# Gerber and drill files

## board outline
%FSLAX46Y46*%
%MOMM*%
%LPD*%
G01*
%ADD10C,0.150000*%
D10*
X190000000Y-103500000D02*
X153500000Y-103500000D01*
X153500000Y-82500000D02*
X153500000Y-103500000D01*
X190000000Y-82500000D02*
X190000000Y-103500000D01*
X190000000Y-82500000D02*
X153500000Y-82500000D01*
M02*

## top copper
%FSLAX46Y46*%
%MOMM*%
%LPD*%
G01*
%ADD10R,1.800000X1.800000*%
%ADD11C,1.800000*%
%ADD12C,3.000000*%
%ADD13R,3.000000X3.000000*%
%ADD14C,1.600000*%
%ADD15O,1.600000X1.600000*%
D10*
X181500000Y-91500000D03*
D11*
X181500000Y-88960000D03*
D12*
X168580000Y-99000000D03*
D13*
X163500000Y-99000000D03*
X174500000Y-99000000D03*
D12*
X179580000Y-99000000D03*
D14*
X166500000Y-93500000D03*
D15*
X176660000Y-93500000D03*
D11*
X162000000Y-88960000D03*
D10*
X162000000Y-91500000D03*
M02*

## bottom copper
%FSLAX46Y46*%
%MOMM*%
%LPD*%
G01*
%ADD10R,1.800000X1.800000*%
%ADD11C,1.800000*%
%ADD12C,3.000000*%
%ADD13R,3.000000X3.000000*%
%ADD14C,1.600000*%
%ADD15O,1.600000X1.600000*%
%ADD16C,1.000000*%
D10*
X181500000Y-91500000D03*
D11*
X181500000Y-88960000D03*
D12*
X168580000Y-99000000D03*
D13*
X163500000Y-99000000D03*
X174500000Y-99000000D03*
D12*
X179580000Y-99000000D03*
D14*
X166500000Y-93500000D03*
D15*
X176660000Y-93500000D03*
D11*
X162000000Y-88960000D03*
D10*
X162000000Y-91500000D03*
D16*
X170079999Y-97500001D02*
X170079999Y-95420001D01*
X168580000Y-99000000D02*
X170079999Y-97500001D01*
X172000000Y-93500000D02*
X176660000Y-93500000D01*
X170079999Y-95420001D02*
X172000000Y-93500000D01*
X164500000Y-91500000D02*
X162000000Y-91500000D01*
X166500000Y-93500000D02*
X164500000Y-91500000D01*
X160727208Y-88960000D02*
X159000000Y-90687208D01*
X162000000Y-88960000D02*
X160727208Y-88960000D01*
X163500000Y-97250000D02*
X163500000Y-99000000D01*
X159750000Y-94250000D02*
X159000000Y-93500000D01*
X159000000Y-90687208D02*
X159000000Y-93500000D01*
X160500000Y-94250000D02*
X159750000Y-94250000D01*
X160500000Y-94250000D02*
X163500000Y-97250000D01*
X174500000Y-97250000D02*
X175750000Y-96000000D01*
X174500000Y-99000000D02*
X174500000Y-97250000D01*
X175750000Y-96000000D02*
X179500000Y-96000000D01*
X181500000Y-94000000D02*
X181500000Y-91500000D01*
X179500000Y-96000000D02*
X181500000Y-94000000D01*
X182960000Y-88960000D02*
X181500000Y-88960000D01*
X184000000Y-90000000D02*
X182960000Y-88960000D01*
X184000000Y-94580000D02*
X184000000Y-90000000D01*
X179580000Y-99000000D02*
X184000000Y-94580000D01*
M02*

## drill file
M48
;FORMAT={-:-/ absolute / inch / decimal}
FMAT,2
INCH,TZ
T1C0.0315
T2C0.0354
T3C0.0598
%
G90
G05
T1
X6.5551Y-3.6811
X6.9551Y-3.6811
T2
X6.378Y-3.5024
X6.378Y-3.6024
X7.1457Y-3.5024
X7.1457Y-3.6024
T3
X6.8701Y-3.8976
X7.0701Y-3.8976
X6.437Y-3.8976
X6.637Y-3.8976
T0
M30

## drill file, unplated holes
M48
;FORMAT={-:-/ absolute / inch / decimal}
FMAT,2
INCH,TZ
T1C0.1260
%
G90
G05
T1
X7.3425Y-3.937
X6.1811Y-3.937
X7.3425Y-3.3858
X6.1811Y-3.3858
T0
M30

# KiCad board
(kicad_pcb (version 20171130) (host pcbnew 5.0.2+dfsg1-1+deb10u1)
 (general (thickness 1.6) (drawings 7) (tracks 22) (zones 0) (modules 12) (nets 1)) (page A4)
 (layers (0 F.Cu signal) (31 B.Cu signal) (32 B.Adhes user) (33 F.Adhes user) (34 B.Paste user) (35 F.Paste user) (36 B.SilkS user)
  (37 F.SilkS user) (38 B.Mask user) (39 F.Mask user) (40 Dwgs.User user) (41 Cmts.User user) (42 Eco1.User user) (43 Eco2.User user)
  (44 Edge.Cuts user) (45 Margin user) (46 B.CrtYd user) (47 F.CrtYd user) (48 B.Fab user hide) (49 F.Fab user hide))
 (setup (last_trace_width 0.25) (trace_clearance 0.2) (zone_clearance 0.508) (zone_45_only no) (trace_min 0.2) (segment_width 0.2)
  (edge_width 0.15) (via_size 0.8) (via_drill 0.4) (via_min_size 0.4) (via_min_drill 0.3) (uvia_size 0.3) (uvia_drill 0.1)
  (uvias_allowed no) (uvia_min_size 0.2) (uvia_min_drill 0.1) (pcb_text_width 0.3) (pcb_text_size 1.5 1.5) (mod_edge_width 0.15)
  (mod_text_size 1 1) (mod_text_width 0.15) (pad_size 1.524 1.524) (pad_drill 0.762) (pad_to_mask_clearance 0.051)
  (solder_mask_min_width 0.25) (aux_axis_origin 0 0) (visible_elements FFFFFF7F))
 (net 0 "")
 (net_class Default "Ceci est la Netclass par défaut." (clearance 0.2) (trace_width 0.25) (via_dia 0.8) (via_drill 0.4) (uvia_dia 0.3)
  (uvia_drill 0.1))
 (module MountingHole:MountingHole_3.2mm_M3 (layer F.Cu) (at 157 100)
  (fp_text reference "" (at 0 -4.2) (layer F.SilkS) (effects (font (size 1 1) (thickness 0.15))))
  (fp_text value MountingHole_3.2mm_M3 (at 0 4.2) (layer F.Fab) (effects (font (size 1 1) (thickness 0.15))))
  (pad 1 np_thru_hole circle (at 0 0) (size 3.2 3.2) (drill 3.2) (layers *.Cu *.Mask)))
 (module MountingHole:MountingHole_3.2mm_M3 (layer F.Cu) (at 186.5 100)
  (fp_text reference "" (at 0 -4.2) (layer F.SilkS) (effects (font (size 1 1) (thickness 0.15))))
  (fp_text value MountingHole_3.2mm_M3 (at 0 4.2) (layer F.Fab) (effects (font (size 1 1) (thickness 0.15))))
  (pad 1 np_thru_hole circle (at 0 0) (size 3.2 3.2) (drill 3.2) (layers *.Cu *.Mask)))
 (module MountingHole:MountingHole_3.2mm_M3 (layer F.Cu) (at 186.5 86)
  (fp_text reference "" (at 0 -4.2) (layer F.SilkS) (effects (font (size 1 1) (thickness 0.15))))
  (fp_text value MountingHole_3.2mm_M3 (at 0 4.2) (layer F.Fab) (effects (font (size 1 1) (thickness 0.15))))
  (pad 1 np_thru_hole circle (at 0 0) (size 3.2 3.2) (drill 3.2) (layers *.Cu *.Mask)))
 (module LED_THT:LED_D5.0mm (layer F.Cu) (at 181.5 91.5 90)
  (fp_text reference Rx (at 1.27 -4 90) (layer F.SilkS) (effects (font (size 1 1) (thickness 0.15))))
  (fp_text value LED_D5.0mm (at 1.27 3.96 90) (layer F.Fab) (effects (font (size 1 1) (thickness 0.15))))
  (pad 1 thru_hole rect (at 0 0 90) (size 1.8 1.8) (drill 0.9) (layers *.Cu *.Mask))
  (pad 2 thru_hole circle (at 2.54 0 90) (size 1.8 1.8) (drill 0.9) (layers *.Cu *.Mask)))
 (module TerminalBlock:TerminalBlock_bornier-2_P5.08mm (layer F.Cu) (at 163.5 99)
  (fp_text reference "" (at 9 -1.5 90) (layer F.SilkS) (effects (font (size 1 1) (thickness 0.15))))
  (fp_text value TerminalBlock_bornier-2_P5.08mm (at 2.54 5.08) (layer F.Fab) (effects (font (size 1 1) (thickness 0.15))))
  (pad 2 thru_hole circle (at 5.08 0) (size 3 3) (drill 1.52) (layers *.Cu *.Mask))
  (pad 1 thru_hole rect (at 0 0) (size 3 3) (drill 1.52) (layers *.Cu *.Mask)))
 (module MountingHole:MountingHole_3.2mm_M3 (layer F.Cu) (at 157 86)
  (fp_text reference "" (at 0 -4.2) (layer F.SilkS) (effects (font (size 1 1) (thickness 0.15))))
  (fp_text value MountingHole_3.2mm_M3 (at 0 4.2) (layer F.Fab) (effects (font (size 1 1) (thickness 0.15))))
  (pad 1 np_thru_hole circle (at 0 0) (size 3.2 3.2) (drill 3.2) (layers *.Cu *.Mask)))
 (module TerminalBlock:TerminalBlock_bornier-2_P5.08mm (layer F.Cu) (at 174.5 99)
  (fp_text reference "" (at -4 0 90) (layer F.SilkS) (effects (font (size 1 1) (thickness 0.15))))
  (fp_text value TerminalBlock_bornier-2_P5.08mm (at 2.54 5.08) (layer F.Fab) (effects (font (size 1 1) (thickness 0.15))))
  (pad 1 thru_hole rect (at 0 0) (size 3 3) (drill 1.52) (layers *.Cu *.Mask))
  (pad 2 thru_hole circle (at 5.08 0) (size 3 3) (drill 1.52) (layers *.Cu *.Mask)))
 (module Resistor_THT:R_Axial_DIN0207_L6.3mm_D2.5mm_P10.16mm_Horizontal (layer F.Cu) (at 166.5 93.5)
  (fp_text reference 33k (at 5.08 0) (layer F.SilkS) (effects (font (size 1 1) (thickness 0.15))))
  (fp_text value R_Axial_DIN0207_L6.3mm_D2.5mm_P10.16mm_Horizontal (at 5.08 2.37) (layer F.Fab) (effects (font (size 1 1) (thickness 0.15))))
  (pad 1 thru_hole circle (at 0 0) (size 1.6 1.6) (drill 0.8) (layers *.Cu *.Mask))
  (pad 2 thru_hole oval (at 10.16 0) (size 1.6 1.6) (drill 0.8) (layers *.Cu *.Mask)))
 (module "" (layer F.Cu) (at 72 144.5)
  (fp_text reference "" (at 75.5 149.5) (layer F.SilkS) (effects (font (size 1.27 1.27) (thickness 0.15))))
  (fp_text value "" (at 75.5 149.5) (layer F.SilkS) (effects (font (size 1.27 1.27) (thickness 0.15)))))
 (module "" (layer F.Cu) (at 45.5 145)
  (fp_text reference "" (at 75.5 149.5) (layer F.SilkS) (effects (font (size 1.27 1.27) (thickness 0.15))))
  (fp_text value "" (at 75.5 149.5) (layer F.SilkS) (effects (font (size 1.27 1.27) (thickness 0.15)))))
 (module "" (layer F.Cu) (at 80 110.5)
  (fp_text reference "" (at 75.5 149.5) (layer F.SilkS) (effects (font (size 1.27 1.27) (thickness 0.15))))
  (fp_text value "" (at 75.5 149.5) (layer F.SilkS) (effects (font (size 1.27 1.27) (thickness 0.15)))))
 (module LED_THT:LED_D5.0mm (layer F.Cu) (at 162 91.5 90)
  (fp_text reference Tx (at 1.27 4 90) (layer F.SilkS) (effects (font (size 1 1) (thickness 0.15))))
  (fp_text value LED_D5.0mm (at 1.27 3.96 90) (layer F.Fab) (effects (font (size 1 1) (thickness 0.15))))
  (pad 2 thru_hole circle (at 2.54 0 90) (size 1.8 1.8) (drill 0.9) (layers *.Cu *.Mask))
  (pad 1 thru_hole rect (at 0 0 90) (size 1.8 1.8) (drill 0.9) (layers *.Cu *.Mask)))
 (gr_line (start 190 103.5) (end 153.5 103.5) (layer Edge.Cuts) (width 0.15))
 (gr_line (start 153.5 82.5) (end 153.5 103.5) (layer Edge.Cuts) (width 0.15))
 (gr_line (start 190 82.5) (end 190 103.5) (layer Edge.Cuts) (width 0.15))
 (gr_line (start 190 82.5) (end 153.5 82.5) (layer Edge.Cuts) (width 0.15))
 (segment (start 170.079999 97.500001) (end 170.079999 95.420001) (width 1) (layer B.Cu) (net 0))
 (segment (start 168.58 99) (end 170.079999 97.500001) (width 1) (layer B.Cu) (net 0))
 (segment (start 172 93.5) (end 176.66 93.5) (width 1) (layer B.Cu) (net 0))
 (segment (start 170.079999 95.420001) (end 172 93.5) (width 1) (layer B.Cu) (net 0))
 (segment (start 164.5 91.5) (end 162 91.5) (width 1) (layer B.Cu) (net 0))
 (segment (start 166.5 93.5) (end 164.5 91.5) (width 1) (layer B.Cu) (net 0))
 (segment (start 160.727208 88.96) (end 159 90.687208) (width 1) (layer B.Cu) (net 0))
 (segment (start 162 88.96) (end 160.727208 88.96) (width 1) (layer B.Cu) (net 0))
 (segment (start 163.5 97.25) (end 163.5 99) (width 1) (layer B.Cu) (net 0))
 (segment (start 159.75 94.25) (end 159 93.5) (width 1) (layer B.Cu) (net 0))
 (segment (start 159 90.687208) (end 159 93.5) (width 1) (layer B.Cu) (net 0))
 (segment (start 160.5 94.25) (end 159.75 94.25) (width 1) (layer B.Cu) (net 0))
 (segment (start 160.5 94.25) (end 163.5 97.25) (width 1) (layer B.Cu) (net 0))
 (segment (start 174.5 97.25) (end 175.75 96) (width 1) (layer B.Cu) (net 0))
 (segment (start 174.5 99) (end 174.5 97.25) (width 1) (layer B.Cu) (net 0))
 (segment (start 175.75 96) (end 179.5 96) (width 1) (layer B.Cu) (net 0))
 (segment (start 181.5 94) (end 181.5 91.5) (width 1) (layer B.Cu) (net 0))
 (segment (start 179.5 96) (end 181.5 94) (width 1) (layer B.Cu) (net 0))
 (segment (start 182.96 88.96) (end 181.5 88.96) (width 1) (layer B.Cu) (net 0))
 (segment (start 184 90) (end 182.96 88.96) (width 1) (layer B.Cu) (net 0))
 (segment (start 184 94.58) (end 184 90) (width 1) (layer B.Cu) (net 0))
 (segment (start 179.58 99) (end 184 94.58) (width 1) (layer B.Cu) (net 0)))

